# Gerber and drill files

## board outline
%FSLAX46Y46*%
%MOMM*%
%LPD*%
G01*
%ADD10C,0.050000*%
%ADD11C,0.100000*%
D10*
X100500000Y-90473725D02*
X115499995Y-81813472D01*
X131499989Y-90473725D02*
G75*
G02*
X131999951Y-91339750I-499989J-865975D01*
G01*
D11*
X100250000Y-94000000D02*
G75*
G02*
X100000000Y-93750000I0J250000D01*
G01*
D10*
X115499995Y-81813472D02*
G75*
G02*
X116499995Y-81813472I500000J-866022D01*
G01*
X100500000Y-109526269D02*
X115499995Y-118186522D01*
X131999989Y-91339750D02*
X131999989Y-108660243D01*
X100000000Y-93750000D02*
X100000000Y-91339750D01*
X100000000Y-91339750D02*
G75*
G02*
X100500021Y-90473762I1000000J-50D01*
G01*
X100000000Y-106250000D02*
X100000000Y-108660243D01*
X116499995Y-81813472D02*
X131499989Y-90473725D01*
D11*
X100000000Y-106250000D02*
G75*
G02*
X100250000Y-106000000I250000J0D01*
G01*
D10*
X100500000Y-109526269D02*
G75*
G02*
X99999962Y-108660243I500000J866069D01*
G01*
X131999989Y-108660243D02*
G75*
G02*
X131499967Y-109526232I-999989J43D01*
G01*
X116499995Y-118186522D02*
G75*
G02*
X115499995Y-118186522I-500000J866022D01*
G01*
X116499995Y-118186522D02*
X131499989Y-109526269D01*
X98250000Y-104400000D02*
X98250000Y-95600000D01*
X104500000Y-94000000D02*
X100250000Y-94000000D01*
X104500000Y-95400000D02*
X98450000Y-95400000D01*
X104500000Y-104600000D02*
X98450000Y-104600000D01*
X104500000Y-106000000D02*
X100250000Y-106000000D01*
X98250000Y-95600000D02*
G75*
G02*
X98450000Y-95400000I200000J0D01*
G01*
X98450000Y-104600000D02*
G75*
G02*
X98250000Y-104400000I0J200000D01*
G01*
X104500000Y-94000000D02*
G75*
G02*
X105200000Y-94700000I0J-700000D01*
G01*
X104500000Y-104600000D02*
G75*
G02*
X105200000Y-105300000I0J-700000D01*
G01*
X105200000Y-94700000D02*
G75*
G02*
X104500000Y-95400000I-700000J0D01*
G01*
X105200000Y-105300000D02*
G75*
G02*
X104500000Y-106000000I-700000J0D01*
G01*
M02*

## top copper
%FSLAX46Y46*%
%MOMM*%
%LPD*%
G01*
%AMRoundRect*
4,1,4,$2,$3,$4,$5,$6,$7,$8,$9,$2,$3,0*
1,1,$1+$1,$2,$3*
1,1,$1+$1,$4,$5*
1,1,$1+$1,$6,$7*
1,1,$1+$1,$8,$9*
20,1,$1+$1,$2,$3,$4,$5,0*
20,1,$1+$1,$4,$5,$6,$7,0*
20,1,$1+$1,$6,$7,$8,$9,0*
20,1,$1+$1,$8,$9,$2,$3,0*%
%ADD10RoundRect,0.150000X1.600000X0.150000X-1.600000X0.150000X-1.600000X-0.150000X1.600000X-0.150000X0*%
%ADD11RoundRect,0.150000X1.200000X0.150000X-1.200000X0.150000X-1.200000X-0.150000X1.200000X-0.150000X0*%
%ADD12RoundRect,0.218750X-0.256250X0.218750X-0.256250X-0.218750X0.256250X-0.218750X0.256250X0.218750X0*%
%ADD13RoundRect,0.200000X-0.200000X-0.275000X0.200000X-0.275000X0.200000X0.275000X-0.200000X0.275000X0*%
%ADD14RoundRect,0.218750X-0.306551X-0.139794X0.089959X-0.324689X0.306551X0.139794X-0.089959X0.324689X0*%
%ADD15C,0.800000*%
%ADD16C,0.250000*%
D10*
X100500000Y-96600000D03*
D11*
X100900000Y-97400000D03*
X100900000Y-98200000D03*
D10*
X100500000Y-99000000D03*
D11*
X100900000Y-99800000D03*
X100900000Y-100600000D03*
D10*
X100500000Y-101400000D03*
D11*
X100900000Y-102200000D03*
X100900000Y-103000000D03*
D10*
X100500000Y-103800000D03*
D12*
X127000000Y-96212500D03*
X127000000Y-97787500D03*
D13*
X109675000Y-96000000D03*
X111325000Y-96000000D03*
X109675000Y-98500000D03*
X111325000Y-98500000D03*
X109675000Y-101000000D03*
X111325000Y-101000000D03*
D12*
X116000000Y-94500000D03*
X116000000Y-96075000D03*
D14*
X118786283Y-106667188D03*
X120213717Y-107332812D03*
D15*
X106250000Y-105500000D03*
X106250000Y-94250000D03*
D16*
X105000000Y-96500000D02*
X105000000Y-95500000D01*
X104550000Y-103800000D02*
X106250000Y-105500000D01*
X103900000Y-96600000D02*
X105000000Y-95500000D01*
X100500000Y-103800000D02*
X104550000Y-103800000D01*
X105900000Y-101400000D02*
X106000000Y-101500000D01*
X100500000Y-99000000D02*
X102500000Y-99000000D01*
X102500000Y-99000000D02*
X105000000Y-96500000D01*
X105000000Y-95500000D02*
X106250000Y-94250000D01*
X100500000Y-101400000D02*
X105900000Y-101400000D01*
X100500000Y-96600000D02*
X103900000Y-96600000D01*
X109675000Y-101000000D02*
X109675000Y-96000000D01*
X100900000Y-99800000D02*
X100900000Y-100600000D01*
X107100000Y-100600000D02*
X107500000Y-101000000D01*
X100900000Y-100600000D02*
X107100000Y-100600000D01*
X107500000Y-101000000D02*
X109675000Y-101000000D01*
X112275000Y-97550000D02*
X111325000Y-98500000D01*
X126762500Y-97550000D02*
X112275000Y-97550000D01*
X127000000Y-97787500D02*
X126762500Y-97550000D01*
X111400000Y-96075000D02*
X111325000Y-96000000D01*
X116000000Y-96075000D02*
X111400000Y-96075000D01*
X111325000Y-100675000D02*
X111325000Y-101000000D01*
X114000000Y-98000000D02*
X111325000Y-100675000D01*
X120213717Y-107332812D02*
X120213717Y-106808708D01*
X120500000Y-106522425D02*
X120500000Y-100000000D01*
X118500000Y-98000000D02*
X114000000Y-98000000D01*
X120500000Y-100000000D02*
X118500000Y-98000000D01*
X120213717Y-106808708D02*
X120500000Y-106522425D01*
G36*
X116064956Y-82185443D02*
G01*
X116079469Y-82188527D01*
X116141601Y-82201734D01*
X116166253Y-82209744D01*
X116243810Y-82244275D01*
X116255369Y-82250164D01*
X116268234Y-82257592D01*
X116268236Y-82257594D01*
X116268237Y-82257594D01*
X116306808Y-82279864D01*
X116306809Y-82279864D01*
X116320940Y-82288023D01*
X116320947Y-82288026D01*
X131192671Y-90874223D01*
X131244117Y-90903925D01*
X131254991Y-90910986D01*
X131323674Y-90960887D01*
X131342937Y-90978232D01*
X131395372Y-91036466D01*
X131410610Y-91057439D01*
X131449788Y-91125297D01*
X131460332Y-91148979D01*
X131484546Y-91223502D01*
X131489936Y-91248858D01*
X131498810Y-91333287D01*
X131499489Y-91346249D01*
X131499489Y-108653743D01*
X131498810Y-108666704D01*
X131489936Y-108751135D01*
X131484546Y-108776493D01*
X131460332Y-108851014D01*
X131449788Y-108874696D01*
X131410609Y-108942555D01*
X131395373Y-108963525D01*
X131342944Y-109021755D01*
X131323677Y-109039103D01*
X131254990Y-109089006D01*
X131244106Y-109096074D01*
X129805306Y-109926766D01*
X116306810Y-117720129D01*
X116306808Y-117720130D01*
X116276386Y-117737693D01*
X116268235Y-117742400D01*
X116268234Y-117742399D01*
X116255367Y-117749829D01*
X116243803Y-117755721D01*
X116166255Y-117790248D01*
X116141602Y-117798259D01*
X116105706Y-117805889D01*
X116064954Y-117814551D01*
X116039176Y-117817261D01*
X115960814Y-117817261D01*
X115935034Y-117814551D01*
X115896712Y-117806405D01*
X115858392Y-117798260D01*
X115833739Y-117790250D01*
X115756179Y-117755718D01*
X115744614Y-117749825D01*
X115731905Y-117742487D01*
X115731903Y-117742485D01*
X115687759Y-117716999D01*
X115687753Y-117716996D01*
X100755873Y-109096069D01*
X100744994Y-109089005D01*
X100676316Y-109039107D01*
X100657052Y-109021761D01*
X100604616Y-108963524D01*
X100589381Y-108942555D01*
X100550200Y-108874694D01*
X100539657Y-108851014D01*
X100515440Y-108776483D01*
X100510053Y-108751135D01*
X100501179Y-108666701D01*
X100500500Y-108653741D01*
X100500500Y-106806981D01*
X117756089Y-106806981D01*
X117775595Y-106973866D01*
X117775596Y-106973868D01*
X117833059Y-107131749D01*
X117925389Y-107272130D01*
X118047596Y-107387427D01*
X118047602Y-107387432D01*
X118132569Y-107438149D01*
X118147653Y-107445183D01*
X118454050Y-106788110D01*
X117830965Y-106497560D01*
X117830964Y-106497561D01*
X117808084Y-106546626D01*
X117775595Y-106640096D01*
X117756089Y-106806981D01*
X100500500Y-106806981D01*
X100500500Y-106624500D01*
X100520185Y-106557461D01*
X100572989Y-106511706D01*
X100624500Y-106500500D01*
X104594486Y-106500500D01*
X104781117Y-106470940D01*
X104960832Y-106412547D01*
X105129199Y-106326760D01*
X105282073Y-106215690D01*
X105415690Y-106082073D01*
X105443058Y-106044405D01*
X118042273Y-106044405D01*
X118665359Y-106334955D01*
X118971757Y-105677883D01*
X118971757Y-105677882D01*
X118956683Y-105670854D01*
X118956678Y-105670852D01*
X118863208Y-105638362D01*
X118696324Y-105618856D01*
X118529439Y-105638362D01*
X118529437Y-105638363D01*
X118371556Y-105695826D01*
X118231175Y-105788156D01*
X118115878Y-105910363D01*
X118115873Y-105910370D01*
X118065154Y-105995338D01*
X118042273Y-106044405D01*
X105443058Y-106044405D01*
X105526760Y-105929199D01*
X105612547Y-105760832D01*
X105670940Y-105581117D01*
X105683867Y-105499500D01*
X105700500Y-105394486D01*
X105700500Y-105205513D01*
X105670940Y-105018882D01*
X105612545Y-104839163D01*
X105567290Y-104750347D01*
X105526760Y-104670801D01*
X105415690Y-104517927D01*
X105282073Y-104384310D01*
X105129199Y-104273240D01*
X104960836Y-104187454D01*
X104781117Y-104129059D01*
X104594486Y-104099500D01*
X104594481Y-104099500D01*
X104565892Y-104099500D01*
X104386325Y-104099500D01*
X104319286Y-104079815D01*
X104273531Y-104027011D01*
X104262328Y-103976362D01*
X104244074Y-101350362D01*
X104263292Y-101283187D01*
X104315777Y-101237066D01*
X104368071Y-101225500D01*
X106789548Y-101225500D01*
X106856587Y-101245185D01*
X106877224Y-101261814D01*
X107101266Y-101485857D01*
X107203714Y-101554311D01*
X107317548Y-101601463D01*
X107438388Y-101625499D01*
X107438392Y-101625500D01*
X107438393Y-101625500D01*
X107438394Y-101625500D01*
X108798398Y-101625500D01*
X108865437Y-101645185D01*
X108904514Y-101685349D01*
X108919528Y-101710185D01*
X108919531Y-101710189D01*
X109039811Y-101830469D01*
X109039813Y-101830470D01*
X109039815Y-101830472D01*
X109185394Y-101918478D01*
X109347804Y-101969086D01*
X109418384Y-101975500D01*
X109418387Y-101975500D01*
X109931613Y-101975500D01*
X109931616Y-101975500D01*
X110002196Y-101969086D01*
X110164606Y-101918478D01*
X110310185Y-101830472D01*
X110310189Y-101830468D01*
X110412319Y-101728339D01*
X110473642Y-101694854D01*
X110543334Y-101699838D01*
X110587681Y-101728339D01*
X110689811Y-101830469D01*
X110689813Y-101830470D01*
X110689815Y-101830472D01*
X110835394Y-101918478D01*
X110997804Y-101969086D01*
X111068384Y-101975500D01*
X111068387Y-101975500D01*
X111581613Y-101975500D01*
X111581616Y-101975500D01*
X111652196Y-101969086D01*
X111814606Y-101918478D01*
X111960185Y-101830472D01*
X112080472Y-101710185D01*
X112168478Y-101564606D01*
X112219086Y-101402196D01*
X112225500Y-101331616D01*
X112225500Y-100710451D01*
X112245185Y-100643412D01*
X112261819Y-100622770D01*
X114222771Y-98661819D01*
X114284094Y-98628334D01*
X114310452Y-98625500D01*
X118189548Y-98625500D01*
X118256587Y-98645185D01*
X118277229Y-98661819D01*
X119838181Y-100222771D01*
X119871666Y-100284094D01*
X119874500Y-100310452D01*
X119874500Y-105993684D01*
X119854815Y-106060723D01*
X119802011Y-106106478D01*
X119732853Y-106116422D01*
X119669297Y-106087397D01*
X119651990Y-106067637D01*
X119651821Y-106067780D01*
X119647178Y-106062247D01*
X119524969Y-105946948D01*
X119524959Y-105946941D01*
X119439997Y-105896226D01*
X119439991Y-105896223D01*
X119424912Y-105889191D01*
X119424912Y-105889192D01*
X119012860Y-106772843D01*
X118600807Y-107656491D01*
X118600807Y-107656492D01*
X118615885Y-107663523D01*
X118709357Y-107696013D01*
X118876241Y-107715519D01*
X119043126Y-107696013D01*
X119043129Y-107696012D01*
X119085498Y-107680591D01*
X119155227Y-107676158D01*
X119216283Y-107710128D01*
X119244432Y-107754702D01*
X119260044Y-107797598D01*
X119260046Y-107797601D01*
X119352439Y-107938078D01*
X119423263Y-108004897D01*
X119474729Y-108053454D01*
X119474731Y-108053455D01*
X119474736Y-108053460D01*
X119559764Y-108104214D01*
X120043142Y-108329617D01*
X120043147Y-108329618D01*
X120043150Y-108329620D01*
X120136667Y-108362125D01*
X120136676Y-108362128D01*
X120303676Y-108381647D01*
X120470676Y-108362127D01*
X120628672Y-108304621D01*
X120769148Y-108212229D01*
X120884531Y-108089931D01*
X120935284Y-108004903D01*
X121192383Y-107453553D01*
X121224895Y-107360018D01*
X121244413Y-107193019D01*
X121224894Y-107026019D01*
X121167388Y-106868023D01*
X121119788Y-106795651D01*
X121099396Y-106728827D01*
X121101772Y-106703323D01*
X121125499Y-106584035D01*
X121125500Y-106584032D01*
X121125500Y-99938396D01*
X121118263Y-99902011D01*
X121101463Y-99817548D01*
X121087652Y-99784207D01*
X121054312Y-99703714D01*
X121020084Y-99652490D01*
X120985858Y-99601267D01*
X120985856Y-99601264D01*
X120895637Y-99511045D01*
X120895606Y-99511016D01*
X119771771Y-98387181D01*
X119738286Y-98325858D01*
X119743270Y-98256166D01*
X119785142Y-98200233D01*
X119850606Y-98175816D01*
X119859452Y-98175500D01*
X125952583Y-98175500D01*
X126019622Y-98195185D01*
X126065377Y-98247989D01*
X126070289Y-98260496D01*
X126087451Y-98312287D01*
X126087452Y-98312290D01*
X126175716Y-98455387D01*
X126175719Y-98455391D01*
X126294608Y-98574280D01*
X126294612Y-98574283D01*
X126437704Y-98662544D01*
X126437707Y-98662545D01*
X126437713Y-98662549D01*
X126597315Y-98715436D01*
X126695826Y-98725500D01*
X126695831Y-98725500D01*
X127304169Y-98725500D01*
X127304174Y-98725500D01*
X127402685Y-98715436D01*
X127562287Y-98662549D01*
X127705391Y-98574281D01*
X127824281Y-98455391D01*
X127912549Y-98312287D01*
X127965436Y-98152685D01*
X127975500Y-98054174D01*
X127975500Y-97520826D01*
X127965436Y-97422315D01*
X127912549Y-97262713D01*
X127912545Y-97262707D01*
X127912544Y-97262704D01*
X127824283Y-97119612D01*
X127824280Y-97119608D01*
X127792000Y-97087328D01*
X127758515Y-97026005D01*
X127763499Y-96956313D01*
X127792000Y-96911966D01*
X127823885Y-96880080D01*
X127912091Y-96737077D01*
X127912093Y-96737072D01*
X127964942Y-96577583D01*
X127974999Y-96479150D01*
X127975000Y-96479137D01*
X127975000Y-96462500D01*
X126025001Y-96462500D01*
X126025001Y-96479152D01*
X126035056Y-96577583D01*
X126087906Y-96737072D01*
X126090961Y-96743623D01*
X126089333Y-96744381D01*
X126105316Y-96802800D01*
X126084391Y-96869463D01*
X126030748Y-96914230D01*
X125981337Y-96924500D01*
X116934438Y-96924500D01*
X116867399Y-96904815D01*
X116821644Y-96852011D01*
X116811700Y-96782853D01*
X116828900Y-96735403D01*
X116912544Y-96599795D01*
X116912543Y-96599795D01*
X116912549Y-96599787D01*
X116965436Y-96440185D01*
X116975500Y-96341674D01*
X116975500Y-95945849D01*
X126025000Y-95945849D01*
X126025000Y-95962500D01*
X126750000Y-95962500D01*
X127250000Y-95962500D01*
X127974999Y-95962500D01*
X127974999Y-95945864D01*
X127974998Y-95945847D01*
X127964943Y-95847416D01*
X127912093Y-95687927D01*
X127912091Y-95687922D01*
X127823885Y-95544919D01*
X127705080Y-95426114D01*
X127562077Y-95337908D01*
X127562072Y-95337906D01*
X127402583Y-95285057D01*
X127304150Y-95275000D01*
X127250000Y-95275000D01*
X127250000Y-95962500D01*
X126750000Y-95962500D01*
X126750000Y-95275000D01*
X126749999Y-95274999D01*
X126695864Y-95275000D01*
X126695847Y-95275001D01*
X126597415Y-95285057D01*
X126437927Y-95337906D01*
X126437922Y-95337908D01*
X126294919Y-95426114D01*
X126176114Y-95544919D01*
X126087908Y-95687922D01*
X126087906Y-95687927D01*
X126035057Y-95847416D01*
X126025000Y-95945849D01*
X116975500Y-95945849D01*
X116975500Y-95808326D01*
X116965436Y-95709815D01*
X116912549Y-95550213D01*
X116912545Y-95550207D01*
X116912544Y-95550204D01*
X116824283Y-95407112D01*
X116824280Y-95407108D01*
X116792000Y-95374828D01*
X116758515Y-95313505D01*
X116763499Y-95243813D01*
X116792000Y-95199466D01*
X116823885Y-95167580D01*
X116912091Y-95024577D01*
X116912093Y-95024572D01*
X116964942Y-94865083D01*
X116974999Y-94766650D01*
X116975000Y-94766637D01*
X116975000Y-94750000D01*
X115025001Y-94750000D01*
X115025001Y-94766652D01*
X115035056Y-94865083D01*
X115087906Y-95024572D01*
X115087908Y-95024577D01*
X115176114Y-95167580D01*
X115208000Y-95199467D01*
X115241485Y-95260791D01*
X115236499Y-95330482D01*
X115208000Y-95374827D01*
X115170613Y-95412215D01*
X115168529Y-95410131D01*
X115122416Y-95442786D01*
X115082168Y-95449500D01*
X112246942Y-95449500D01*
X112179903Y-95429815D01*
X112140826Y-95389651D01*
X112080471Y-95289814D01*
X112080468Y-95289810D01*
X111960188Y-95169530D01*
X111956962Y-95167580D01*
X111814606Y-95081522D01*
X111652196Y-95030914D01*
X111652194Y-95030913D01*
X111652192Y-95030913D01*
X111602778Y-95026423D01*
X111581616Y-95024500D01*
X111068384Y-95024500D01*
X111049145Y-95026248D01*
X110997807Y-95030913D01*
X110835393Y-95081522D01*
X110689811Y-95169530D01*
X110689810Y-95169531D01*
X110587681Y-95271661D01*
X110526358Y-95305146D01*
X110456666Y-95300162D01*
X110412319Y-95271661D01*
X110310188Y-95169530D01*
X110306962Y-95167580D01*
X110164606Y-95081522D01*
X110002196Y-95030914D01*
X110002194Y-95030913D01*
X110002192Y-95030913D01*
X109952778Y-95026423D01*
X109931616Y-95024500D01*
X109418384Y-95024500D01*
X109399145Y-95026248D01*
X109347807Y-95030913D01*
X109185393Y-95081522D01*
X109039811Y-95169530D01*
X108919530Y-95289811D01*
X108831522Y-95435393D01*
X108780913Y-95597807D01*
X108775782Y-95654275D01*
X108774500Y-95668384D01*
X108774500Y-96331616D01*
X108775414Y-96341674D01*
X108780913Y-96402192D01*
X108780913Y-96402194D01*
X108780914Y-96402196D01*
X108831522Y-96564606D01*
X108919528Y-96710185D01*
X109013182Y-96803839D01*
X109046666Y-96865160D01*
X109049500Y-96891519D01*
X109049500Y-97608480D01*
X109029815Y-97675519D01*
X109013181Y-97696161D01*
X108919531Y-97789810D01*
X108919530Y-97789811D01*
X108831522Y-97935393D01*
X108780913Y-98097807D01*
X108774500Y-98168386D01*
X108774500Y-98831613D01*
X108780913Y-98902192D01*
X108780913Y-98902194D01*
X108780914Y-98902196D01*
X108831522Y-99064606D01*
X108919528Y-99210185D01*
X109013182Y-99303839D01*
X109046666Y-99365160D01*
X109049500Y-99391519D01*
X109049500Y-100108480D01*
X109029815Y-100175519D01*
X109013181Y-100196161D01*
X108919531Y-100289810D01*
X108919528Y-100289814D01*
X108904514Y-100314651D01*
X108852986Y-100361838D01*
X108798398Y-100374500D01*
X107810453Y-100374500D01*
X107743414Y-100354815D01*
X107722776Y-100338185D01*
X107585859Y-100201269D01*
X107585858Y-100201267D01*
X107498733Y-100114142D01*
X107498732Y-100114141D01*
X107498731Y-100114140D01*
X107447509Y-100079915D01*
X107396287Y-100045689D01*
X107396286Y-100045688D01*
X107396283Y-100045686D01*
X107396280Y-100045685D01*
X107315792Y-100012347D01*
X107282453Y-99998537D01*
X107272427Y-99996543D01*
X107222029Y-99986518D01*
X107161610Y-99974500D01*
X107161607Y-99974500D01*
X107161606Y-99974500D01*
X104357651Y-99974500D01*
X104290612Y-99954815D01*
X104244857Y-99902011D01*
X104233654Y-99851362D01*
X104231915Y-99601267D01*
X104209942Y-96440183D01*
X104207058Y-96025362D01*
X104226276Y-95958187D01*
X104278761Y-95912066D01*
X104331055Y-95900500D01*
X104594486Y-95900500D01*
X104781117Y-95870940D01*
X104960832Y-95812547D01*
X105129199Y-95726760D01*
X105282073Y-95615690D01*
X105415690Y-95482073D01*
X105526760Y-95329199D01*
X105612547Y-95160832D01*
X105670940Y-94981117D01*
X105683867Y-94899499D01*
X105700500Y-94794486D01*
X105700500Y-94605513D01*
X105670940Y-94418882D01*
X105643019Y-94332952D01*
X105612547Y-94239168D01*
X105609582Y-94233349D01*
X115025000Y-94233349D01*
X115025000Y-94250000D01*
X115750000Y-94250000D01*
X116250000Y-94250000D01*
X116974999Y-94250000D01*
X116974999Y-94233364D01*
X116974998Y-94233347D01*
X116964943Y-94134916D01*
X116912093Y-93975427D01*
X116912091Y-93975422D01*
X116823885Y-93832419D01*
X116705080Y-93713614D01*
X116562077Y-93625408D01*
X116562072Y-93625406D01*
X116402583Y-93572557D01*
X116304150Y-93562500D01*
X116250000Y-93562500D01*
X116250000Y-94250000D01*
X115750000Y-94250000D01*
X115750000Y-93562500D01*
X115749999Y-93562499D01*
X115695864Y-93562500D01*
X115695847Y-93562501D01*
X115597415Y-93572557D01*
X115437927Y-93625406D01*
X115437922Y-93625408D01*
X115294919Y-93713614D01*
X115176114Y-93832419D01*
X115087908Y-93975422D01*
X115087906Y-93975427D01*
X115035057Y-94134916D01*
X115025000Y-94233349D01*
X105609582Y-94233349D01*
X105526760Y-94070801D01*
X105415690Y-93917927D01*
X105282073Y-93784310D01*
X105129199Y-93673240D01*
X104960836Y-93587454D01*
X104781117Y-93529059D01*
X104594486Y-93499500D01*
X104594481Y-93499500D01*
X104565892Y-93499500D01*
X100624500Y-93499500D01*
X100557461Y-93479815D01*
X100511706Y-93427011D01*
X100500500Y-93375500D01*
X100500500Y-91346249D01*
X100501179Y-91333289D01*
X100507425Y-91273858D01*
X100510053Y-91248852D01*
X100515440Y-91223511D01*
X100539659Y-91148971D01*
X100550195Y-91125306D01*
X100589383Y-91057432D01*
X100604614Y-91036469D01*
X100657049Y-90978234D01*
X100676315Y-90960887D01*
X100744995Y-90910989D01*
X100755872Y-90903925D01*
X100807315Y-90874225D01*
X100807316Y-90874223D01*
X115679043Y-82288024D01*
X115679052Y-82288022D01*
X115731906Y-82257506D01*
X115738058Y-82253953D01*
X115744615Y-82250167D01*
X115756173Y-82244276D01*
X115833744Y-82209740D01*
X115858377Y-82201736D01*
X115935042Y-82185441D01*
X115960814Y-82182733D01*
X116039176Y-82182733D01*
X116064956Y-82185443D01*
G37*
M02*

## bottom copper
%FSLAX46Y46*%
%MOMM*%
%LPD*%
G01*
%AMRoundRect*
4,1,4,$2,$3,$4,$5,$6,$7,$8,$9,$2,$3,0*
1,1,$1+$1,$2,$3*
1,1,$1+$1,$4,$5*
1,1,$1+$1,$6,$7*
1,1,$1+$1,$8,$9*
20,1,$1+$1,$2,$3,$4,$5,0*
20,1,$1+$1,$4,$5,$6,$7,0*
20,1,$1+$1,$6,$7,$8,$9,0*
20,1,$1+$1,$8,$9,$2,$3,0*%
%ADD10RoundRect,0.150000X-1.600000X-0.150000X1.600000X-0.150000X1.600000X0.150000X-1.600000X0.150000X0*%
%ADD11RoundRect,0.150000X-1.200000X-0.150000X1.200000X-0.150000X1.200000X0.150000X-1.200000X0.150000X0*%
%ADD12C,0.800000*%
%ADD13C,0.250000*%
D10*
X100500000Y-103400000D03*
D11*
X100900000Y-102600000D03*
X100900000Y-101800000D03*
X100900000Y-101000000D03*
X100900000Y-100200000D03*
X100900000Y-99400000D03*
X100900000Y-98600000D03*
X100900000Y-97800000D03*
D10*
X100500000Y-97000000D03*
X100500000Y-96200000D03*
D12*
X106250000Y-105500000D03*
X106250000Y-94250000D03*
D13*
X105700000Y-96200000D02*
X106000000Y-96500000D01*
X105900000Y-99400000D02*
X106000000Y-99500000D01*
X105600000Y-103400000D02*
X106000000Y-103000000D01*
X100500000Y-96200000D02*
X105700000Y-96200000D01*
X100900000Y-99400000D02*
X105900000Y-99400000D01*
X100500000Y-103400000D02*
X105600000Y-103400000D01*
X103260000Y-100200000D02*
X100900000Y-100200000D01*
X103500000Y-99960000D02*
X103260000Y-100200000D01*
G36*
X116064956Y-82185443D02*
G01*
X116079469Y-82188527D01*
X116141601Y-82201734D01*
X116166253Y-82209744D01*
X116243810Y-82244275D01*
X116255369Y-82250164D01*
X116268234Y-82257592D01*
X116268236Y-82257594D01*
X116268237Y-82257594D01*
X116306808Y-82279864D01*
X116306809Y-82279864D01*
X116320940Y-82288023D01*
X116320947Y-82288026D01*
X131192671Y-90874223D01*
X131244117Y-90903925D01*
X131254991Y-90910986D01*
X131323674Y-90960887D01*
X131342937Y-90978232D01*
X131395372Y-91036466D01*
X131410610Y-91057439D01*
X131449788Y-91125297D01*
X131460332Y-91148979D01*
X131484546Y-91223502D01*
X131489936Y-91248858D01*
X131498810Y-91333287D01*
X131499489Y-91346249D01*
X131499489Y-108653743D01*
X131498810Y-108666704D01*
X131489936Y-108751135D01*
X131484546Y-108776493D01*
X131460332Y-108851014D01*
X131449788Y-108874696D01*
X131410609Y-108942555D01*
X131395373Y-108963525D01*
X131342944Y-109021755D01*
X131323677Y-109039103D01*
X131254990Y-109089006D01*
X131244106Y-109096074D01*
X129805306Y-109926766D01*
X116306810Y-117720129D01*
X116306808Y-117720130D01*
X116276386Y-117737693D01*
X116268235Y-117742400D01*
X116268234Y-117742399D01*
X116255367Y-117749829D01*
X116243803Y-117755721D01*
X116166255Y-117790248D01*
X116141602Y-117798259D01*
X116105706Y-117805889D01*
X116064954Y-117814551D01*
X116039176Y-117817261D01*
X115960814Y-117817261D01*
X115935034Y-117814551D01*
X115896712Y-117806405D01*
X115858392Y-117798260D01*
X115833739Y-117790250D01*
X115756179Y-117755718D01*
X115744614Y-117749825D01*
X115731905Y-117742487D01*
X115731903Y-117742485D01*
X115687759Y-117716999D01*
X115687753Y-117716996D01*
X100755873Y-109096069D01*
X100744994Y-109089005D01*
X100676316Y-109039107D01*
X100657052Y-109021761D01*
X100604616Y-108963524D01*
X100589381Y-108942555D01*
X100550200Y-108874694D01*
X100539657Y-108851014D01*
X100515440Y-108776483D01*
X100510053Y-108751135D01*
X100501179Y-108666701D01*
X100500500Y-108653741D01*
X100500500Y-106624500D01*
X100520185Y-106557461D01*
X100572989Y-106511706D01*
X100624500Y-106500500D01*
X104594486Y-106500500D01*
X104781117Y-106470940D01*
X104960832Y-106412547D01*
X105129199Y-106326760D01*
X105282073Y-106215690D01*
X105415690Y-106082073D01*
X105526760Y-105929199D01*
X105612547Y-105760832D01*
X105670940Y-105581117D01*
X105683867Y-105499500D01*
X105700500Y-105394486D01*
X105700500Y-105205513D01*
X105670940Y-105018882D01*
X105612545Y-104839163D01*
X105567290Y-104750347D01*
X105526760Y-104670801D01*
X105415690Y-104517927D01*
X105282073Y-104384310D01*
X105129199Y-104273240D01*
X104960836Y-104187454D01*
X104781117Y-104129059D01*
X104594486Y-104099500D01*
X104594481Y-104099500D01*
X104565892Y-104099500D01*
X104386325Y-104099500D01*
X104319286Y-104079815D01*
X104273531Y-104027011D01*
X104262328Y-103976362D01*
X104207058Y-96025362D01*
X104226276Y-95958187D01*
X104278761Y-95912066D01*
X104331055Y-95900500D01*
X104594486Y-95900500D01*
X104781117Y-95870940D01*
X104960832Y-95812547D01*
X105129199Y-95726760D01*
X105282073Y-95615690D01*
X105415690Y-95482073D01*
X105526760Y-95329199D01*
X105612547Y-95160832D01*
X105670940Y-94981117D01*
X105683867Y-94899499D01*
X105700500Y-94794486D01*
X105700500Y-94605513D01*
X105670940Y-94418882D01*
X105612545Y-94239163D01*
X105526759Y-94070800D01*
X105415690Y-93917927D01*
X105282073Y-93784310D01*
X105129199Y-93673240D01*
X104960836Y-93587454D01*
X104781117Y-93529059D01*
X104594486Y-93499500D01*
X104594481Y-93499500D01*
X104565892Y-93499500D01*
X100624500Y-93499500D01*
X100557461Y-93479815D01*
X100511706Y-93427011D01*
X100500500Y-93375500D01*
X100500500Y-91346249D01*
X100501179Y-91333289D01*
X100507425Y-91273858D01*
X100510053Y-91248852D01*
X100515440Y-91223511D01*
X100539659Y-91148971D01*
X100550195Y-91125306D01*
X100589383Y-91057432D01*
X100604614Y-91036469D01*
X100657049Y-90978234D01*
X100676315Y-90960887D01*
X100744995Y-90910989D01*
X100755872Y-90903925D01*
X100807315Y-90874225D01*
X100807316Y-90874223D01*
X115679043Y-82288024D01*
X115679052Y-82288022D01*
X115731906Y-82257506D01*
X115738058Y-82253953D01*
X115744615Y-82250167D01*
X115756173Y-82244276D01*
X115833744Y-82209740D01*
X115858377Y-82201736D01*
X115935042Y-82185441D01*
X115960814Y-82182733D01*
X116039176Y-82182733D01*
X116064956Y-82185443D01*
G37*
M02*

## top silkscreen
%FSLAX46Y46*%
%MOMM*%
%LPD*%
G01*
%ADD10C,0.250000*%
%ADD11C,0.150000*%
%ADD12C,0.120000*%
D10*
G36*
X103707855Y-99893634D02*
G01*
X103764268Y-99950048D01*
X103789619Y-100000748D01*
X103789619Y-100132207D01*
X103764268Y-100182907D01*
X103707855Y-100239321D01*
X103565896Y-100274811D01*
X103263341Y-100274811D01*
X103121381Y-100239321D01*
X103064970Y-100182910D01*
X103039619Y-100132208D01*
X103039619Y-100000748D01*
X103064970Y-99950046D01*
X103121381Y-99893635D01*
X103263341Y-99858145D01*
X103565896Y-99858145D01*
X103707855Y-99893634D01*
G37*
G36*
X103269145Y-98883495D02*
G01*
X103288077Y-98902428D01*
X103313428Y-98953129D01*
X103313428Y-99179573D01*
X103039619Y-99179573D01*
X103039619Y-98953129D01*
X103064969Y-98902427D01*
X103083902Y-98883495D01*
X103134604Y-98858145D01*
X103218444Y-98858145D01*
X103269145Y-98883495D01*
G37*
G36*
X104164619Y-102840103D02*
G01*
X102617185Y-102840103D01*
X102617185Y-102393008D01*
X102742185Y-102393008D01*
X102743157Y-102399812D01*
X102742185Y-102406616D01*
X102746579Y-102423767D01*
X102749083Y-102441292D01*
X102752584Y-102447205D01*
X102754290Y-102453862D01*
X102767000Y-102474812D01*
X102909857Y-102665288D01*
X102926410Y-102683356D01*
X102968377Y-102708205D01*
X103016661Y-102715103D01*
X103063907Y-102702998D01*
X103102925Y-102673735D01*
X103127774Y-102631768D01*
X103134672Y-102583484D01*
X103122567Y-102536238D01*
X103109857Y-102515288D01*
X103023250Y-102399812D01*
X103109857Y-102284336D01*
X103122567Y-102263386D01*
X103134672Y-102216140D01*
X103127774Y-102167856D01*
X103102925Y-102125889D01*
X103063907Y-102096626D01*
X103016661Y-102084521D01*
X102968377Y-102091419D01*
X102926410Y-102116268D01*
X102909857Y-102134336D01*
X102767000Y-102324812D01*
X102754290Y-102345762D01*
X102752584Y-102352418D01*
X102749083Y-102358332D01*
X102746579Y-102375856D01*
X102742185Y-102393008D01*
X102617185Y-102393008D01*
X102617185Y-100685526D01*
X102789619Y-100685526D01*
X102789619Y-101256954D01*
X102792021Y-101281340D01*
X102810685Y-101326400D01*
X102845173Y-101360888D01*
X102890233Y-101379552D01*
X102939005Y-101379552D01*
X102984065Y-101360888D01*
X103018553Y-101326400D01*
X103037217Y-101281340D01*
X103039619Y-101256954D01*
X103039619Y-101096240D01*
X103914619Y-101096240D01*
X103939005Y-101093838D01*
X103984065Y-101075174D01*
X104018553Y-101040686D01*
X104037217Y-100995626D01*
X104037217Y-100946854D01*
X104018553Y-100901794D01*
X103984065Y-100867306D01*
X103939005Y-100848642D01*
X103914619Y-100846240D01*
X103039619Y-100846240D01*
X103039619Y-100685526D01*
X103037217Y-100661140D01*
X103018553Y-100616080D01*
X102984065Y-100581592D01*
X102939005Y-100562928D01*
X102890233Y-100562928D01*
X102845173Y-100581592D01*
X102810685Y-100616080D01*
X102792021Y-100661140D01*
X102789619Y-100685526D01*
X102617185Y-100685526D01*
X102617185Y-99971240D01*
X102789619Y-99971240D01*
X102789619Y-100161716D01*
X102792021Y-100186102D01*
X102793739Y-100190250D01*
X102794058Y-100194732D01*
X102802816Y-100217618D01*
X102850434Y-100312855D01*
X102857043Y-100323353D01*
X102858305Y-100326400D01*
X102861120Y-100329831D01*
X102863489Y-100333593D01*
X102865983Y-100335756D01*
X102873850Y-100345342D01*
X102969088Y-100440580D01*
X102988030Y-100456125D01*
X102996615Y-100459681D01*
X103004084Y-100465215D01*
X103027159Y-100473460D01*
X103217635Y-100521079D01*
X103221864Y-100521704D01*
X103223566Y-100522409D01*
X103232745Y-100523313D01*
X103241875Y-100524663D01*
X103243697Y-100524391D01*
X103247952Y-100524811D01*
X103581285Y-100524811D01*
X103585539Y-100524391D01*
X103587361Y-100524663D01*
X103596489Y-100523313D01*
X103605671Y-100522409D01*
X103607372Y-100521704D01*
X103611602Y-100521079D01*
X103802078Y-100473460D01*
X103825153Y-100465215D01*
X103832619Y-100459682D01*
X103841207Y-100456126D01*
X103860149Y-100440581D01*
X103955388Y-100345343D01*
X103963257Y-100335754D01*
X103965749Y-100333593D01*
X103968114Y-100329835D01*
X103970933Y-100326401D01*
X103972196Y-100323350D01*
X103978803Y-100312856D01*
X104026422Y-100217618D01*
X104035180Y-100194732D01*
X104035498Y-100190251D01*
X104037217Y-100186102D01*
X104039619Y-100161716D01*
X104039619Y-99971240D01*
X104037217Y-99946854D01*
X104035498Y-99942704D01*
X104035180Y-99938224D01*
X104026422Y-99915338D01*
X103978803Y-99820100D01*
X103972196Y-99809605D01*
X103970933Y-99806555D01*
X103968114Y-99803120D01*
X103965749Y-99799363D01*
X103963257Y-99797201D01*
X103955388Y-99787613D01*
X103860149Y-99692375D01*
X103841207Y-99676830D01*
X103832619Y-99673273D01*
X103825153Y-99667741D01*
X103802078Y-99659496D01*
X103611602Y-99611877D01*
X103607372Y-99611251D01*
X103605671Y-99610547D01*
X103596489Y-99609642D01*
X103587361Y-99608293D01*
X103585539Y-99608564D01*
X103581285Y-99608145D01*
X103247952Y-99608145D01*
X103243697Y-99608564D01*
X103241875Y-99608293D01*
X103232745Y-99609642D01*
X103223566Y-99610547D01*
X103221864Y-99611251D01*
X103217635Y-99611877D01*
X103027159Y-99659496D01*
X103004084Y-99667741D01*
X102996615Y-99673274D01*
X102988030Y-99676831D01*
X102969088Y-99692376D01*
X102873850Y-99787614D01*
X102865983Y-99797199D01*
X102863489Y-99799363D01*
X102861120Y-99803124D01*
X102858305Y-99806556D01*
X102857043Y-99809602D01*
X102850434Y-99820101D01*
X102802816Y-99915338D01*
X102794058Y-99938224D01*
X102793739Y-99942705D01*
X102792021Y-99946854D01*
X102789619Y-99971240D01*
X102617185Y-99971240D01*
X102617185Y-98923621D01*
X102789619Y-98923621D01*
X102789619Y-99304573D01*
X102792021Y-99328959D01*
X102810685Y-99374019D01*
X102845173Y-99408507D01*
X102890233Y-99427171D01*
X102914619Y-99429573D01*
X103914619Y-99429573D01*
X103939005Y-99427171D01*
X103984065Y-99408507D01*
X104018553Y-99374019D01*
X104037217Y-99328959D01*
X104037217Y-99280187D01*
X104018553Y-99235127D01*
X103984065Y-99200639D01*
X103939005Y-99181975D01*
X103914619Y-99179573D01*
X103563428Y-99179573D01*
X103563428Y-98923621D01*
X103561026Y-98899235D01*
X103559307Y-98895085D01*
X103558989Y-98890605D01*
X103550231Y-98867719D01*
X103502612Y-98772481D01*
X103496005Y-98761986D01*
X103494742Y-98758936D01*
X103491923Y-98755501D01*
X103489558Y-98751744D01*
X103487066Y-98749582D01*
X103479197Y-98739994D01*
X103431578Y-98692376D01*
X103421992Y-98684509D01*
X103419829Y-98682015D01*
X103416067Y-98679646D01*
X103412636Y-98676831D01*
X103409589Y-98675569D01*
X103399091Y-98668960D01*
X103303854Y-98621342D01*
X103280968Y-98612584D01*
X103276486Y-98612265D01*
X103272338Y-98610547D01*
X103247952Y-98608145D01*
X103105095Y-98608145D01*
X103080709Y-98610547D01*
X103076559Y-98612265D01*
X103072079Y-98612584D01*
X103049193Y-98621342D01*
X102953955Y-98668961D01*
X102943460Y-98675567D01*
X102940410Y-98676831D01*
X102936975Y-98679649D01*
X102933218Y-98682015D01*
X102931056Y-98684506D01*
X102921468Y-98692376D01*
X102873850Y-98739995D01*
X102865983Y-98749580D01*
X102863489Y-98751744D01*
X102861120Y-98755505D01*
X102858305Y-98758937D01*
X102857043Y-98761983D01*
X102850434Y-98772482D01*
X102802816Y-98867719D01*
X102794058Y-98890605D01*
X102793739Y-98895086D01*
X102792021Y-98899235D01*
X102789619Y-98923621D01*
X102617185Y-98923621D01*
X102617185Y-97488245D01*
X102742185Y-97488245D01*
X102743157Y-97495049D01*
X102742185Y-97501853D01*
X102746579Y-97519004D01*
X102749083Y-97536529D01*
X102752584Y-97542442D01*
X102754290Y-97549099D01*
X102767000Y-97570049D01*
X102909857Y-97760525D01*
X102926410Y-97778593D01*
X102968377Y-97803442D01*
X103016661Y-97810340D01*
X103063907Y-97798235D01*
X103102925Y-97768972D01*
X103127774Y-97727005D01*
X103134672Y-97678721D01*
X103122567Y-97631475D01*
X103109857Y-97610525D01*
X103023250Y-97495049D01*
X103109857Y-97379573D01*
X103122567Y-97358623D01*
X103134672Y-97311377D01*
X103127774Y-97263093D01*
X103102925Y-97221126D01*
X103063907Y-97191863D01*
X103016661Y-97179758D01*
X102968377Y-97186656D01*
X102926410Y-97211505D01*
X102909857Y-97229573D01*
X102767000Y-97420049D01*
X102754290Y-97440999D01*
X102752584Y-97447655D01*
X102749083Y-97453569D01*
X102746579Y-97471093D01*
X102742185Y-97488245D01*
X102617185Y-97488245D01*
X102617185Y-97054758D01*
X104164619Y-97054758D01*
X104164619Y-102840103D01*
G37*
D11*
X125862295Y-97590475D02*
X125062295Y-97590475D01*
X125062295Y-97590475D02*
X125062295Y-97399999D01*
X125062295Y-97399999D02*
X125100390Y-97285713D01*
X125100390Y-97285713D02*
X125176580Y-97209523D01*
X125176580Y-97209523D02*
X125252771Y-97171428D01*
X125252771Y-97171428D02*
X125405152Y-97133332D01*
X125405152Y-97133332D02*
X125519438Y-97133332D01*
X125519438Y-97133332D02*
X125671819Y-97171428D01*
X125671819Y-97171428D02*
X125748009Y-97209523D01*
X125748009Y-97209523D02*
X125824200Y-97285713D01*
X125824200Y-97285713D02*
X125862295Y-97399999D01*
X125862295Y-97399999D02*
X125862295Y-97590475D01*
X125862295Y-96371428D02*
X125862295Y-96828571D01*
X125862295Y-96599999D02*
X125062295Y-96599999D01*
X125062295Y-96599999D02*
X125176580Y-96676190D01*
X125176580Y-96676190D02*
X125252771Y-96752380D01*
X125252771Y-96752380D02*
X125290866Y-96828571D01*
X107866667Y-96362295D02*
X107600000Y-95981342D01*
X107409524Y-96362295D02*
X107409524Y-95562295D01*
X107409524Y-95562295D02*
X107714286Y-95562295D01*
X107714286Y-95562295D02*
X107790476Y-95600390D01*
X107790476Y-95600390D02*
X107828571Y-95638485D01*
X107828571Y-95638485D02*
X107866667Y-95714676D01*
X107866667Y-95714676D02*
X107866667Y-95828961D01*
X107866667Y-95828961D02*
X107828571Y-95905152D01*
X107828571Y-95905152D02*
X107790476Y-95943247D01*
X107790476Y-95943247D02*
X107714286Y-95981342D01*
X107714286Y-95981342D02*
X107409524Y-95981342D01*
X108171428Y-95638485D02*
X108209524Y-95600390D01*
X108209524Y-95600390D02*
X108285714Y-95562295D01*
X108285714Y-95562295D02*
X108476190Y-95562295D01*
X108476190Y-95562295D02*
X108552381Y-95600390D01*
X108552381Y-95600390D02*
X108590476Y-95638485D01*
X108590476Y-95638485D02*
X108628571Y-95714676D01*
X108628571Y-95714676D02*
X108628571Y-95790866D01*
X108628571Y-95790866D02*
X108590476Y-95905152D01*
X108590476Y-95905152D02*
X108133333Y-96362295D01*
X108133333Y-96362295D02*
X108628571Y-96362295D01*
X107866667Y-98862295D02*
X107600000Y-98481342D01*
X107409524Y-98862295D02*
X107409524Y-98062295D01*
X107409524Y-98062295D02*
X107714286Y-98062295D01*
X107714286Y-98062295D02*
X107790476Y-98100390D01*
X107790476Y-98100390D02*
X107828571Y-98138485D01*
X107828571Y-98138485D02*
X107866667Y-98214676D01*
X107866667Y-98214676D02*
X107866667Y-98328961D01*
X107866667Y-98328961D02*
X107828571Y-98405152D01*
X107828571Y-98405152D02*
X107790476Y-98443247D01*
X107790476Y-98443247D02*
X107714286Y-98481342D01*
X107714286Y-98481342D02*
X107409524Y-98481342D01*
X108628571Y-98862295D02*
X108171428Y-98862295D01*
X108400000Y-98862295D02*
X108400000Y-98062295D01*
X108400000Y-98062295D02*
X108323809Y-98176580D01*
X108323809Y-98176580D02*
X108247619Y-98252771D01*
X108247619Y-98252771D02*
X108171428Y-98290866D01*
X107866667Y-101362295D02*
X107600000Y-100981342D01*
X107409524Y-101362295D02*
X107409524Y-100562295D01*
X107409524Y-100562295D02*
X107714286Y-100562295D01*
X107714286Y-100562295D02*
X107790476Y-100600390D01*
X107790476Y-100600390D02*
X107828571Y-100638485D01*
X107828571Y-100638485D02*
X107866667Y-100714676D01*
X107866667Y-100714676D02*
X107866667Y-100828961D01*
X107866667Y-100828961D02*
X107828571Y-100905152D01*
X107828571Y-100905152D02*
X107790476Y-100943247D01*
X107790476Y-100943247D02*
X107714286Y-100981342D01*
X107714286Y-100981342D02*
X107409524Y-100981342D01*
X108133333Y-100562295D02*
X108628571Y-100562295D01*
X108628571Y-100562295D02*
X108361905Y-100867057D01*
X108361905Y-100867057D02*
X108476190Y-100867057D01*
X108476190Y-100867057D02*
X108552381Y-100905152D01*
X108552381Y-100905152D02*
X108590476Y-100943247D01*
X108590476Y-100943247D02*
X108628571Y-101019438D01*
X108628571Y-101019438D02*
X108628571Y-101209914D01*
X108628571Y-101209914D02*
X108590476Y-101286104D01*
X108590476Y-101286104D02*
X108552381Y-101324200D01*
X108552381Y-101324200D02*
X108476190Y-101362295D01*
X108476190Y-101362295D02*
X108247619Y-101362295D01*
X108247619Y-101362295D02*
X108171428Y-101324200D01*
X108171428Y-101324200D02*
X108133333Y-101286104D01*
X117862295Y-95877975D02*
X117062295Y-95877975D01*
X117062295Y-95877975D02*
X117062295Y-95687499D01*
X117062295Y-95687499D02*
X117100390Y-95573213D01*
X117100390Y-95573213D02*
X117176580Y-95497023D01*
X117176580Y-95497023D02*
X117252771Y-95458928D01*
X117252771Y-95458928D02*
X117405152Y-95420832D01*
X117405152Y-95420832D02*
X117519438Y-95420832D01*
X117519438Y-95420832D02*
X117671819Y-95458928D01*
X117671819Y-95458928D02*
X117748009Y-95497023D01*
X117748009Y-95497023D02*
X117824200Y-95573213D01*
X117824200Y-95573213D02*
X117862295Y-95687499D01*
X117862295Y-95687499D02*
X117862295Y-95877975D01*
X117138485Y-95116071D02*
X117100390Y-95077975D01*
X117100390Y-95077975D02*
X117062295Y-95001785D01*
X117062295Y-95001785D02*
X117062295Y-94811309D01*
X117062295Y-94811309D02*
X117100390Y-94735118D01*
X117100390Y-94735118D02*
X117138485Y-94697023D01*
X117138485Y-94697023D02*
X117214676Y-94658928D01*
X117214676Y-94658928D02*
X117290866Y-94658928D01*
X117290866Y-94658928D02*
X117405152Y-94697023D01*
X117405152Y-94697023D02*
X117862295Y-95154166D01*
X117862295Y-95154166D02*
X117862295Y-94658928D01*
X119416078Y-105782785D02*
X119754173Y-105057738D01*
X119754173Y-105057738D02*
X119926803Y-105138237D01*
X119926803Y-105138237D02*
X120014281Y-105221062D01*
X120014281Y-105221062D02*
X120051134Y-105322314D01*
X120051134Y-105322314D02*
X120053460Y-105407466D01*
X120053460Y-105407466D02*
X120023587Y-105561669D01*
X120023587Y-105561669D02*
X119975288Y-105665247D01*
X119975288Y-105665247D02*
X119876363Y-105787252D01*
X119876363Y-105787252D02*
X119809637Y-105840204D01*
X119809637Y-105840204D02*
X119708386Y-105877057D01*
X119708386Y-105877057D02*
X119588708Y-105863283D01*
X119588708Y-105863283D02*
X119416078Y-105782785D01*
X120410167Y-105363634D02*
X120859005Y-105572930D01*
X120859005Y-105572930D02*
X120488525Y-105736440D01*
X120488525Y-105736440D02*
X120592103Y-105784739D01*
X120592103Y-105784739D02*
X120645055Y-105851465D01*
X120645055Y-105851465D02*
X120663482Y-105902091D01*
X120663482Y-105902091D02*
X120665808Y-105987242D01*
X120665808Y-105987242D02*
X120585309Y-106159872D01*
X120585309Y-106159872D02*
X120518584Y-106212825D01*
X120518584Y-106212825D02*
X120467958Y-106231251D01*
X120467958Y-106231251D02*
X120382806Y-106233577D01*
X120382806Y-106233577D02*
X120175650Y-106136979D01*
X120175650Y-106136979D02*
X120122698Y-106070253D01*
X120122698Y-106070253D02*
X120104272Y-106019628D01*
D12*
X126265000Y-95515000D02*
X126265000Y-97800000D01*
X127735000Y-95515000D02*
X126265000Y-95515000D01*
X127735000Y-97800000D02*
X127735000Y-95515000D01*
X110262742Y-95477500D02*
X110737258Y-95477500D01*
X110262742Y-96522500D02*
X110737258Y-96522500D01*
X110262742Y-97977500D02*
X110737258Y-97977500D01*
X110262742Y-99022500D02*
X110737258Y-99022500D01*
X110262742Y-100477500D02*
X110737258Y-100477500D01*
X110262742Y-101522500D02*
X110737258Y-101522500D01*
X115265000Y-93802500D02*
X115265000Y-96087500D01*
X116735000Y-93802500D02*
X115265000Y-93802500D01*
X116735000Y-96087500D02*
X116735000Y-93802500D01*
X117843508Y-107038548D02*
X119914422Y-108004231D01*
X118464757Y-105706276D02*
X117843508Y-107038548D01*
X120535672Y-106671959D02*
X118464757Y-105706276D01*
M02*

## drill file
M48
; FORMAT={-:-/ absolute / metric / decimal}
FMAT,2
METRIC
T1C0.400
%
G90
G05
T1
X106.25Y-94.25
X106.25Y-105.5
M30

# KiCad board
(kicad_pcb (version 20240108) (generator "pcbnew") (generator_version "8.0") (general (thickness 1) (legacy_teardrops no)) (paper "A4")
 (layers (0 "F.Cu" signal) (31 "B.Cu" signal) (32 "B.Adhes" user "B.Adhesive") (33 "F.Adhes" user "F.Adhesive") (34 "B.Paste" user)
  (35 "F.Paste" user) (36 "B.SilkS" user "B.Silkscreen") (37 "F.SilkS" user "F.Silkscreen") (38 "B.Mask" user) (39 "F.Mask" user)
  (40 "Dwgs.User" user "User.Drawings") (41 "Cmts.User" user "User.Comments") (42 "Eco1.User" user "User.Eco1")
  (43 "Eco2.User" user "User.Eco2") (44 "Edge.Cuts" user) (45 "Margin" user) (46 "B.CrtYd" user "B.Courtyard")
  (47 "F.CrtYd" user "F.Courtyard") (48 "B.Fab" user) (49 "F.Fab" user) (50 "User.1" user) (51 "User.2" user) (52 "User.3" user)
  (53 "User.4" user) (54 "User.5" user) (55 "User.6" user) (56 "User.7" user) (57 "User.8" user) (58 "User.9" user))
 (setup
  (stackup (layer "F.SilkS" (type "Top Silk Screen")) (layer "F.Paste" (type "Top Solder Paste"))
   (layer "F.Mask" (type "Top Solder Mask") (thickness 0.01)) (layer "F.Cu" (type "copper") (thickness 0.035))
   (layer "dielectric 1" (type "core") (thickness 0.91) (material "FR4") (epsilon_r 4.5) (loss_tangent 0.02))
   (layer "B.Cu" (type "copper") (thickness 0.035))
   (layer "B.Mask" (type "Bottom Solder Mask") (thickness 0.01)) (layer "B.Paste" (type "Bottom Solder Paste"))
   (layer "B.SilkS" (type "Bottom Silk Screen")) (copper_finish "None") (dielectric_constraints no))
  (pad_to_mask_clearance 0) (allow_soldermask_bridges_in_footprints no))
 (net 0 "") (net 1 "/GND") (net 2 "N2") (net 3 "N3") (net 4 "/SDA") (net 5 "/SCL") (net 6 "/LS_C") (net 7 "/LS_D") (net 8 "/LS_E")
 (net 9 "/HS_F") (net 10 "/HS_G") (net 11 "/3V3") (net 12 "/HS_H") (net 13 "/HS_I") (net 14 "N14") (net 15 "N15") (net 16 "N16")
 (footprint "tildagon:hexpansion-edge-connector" (layer "F.Cu") (at 98.25 100)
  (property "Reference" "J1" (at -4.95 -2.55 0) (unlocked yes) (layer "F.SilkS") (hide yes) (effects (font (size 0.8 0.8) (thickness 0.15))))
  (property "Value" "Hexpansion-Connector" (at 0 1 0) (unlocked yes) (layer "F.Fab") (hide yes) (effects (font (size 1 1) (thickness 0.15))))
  (fp_line (start 0 4.4) (end 0 -4.4) (stroke (width 0.05) (type solid)) (layer "Edge.Cuts"))
  (fp_line (start 6.25 -6) (end 2 -6) (stroke (width 0.05) (type solid)) (layer "Edge.Cuts"))
  (fp_line (start 6.25 -4.6) (end 0.2 -4.6) (stroke (width 0.05) (type solid)) (layer "Edge.Cuts"))
  (fp_line (start 6.25 4.6) (end 0.2 4.6) (stroke (width 0.05) (type solid)) (layer "Edge.Cuts"))
  (fp_line (start 6.25 6) (end 2 6) (stroke (width 0.05) (type solid)) (layer "Edge.Cuts"))
  (fp_arc (start 0 -4.4) (mid 0.058579 -4.541421) (end 0.2 -4.6) (stroke (width 0.05) (type default)) (layer "Edge.Cuts"))
  (fp_arc (start 0.2 4.6) (mid 0.058579 4.541421) (end 0 4.4) (stroke (width 0.05) (type default)) (layer "Edge.Cuts"))
  (fp_arc (start 6.25 -6) (mid 6.744975 -5.794975) (end 6.95 -5.3) (stroke (width 0.05) (type default)) (layer "Edge.Cuts"))
  (fp_arc (start 6.25 4.6) (mid 6.744975 4.805025) (end 6.95 5.3) (stroke (width 0.05) (type default)) (layer "Edge.Cuts"))
  (fp_arc (start 6.95 -5.3) (mid 6.744975 -4.805025) (end 6.25 -4.6) (stroke (width 0.05) (type default)) (layer "Edge.Cuts"))
  (fp_arc (start 6.95 5.3) (mid 6.744975 5.794975) (end 6.25 6) (stroke (width 0.05) (type default)) (layer "Edge.Cuts"))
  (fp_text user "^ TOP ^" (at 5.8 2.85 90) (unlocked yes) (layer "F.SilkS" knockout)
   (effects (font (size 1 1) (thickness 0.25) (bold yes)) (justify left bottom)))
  (pad "1" smd roundrect (at 2.25 3.4) (size 3.5 0.6) (layers "B.Cu" "B.Mask") (roundrect_rratio 0.25) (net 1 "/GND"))
  (pad "2" smd roundrect (at 2.65 2.6) (size 2.7 0.6) (layers "B.Cu" "B.Mask") (roundrect_rratio 0.25) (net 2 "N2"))
  (pad "3" smd roundrect (at 2.65 1.8) (size 2.7 0.6) (layers "B.Cu" "B.Mask") (roundrect_rratio 0.25) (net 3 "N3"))
  (pad "4" smd roundrect (at 2.65 1) (size 2.7 0.6) (layers "B.Cu" "B.Mask") (roundrect_rratio 0.25) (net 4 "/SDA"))
  (pad "5" smd roundrect (at 2.65 0.2) (size 2.7 0.6) (layers "B.Cu" "B.Mask") (roundrect_rratio 0.25) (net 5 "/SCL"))
  (pad "6" smd roundrect (at 2.65 -0.6) (size 2.7 0.6) (layers "B.Cu" "B.Mask") (roundrect_rratio 0.25) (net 1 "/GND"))
  (pad "7" smd roundrect (at 2.65 -1.4) (size 2.7 0.6) (layers "B.Cu" "B.Mask") (roundrect_rratio 0.25) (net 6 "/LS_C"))
  (pad "8" smd roundrect (at 2.65 -2.2) (size 2.7 0.6) (layers "B.Cu" "B.Mask") (roundrect_rratio 0.25) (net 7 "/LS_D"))
  (pad "9" smd roundrect (at 2.25 -3) (size 3.5 0.6) (layers "B.Cu" "B.Mask") (roundrect_rratio 0.25) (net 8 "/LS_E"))
  (pad "10" smd roundrect (at 2.25 -3.8) (size 3.5 0.6) (layers "B.Cu" "B.Mask") (roundrect_rratio 0.25) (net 1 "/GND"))
  (pad "11" smd roundrect (at 2.25 -3.4 180) (size 3.5 0.6) (layers "F.Cu" "F.Mask") (roundrect_rratio 0.25) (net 1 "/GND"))
  (pad "12" smd roundrect (at 2.65 -2.6 180) (size 2.7 0.6) (layers "F.Cu" "F.Mask") (roundrect_rratio 0.25) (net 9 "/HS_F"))
  (pad "13" smd roundrect (at 2.65 -1.8 180) (size 2.7 0.6) (layers "F.Cu" "F.Mask") (roundrect_rratio 0.25) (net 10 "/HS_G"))
  (pad "14" smd roundrect (at 2.25 -1 180) (size 3.5 0.6) (layers "F.Cu" "F.Mask") (roundrect_rratio 0.25) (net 1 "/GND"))
  (pad "15" smd roundrect (at 2.65 -0.2 180) (size 2.7 0.6) (layers "F.Cu" "F.Mask") (roundrect_rratio 0.25) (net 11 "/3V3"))
  (pad "16" smd roundrect (at 2.65 0.6 180) (size 2.7 0.6) (layers "F.Cu" "F.Mask") (roundrect_rratio 0.25) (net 11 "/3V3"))
  (pad "17" smd roundrect (at 2.25 1.4 180) (size 3.5 0.6) (layers "F.Cu" "F.Mask") (roundrect_rratio 0.25) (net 1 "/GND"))
  (pad "18" smd roundrect (at 2.65 2.2 180) (size 2.7 0.6) (layers "F.Cu" "F.Mask") (roundrect_rratio 0.25) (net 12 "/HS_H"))
  (pad "19" smd roundrect (at 2.65 3 180) (size 2.7 0.6) (layers "F.Cu" "F.Mask") (roundrect_rratio 0.25) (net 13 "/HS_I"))
  (pad "20" smd roundrect (at 2.25 3.8 180) (size 3.5 0.6) (layers "F.Cu" "F.Mask") (roundrect_rratio 0.25) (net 1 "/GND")))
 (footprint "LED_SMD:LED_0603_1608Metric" (layer "F.Cu") (at 127 97 -90)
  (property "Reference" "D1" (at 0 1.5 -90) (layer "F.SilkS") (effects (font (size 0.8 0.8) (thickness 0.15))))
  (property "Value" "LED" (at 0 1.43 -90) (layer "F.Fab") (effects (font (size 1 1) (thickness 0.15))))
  (fp_line (start -1.485 0.735) (end 0.8 0.735) (stroke (width 0.12) (type solid)) (layer "F.SilkS"))
  (fp_line (start -1.485 -0.735) (end -1.485 0.735) (stroke (width 0.12) (type solid)) (layer "F.SilkS"))
  (fp_line (start 0.8 -0.735) (end -1.485 -0.735) (stroke (width 0.12) (type solid)) (layer "F.SilkS"))
  (pad "1" smd roundrect (at -0.7875 0 270) (size 0.875 0.95) (layers "F.Cu" "F.Paste" "F.Mask") (roundrect_rratio 0.25) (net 1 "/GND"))
  (pad "2" smd roundrect (at 0.7875 0 270) (size 0.875 0.95) (layers "F.Cu" "F.Paste" "F.Mask") (roundrect_rratio 0.25) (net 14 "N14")))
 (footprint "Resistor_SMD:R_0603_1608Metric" (layer "F.Cu") (at 110.5 96)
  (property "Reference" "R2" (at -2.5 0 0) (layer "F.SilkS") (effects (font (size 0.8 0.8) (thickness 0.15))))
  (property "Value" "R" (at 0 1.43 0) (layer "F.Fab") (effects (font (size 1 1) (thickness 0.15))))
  (fp_line (start -0.237258 -0.5225) (end 0.237258 -0.5225) (stroke (width 0.12) (type solid)) (layer "F.SilkS"))
  (fp_line (start -0.237258 0.5225) (end 0.237258 0.5225) (stroke (width 0.12) (type solid)) (layer "F.SilkS"))
  (pad "1" smd roundrect (at -0.825 0) (size 0.8 0.95) (layers "F.Cu" "F.Paste" "F.Mask") (roundrect_rratio 0.25) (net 11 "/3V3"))
  (pad "2" smd roundrect (at 0.825 0) (size 0.8 0.95) (layers "F.Cu" "F.Paste" "F.Mask") (roundrect_rratio 0.25) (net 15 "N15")))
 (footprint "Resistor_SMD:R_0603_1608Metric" (layer "F.Cu") (at 110.5 98.5)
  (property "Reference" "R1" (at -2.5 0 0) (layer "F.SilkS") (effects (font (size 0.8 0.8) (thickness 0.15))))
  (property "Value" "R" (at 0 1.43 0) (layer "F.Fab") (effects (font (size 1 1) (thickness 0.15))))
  (fp_line (start -0.237258 -0.5225) (end 0.237258 -0.5225) (stroke (width 0.12) (type solid)) (layer "F.SilkS"))
  (fp_line (start -0.237258 0.5225) (end 0.237258 0.5225) (stroke (width 0.12) (type solid)) (layer "F.SilkS"))
  (pad "1" smd roundrect (at -0.825 0) (size 0.8 0.95) (layers "F.Cu" "F.Paste" "F.Mask") (roundrect_rratio 0.25) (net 11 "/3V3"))
  (pad "2" smd roundrect (at 0.825 0) (size 0.8 0.95) (layers "F.Cu" "F.Paste" "F.Mask") (roundrect_rratio 0.25) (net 14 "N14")))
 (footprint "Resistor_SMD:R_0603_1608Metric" (layer "F.Cu") (at 110.5 101)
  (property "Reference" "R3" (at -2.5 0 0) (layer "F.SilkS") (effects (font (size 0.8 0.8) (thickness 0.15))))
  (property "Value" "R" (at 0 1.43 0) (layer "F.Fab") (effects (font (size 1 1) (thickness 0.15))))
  (fp_line (start -0.237258 -0.5225) (end 0.237258 -0.5225) (stroke (width 0.12) (type solid)) (layer "F.SilkS"))
  (fp_line (start -0.237258 0.5225) (end 0.237258 0.5225) (stroke (width 0.12) (type solid)) (layer "F.SilkS"))
  (pad "1" smd roundrect (at -0.825 0) (size 0.8 0.95) (layers "F.Cu" "F.Paste" "F.Mask") (roundrect_rratio 0.25) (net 11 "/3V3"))
  (pad "2" smd roundrect (at 0.825 0) (size 0.8 0.95) (layers "F.Cu" "F.Paste" "F.Mask") (roundrect_rratio 0.25) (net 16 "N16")))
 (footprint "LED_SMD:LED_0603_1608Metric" (layer "F.Cu") (at 116 95.2875 -90)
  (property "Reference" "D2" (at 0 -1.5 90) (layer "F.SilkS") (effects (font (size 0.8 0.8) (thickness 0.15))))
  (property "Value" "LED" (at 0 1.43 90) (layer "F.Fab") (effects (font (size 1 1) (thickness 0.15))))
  (fp_line (start -1.485 0.735) (end 0.8 0.735) (stroke (width 0.12) (type solid)) (layer "F.SilkS"))
  (fp_line (start -1.485 -0.735) (end -1.485 0.735) (stroke (width 0.12) (type solid)) (layer "F.SilkS"))
  (fp_line (start 0.8 -0.735) (end -1.485 -0.735) (stroke (width 0.12) (type solid)) (layer "F.SilkS"))
  (pad "1" smd roundrect (at -0.7875 0 270) (size 0.875 0.95) (layers "F.Cu" "F.Paste" "F.Mask") (roundrect_rratio 0.25) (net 1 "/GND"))
  (pad "2" smd roundrect (at 0.7875 0 270) (size 0.875 0.95) (layers "F.Cu" "F.Paste" "F.Mask") (roundrect_rratio 0.25) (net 15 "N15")))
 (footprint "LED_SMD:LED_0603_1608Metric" (layer "F.Cu") (at 119.5 107 -25)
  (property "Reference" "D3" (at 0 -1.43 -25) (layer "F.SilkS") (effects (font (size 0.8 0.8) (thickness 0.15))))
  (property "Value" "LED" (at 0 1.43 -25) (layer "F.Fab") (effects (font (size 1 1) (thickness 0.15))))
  (fp_line (start -1.485001 0.735) (end 0.8 0.735) (stroke (width 0.12) (type solid)) (layer "F.SilkS"))
  (fp_line (start -1.485 -0.735) (end -1.485001 0.735) (stroke (width 0.12) (type solid)) (layer "F.SilkS"))
  (fp_line (start 0.800001 -0.735) (end -1.485 -0.735) (stroke (width 0.12) (type solid)) (layer "F.SilkS"))
  (pad "1" smd roundrect (at -0.7875 0 335) (size 0.875 0.95) (layers "F.Cu" "F.Paste" "F.Mask") (roundrect_rratio 0.25) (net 1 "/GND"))
  (pad "2" smd roundrect (at 0.7875 0 335) (size 0.875 0.95) (layers "F.Cu" "F.Paste" "F.Mask") (roundrect_rratio 0.25) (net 16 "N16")))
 (gr_line (start 100.5 90.473725) (end 115.499995 81.813472) (stroke (width 0.05) (type solid)) (layer "Edge.Cuts"))
 (gr_arc (start 131.499989 90.473725) (mid 131.866015 90.83975) (end 131.999989 91.33975) (stroke (width 0.05) (type solid))
  (layer "Edge.Cuts"))
 (gr_arc (start 100.25 94) (mid 100.073223 93.926777) (end 100 93.75) (stroke (width 0.1) (type default)) (layer "Edge.Cuts"))
 (gr_arc (start 115.499995 81.813472) (mid 115.999995 81.679497) (end 116.499995 81.813472) (stroke (width 0.05) (type solid))
  (layer "Edge.Cuts"))
 (gr_line (start 100.5 109.526269) (end 115.499995 118.186522) (stroke (width 0.05) (type solid)) (layer "Edge.Cuts"))
 (gr_line (start 131.999989 91.33975) (end 131.999989 108.660243) (stroke (width 0.05) (type solid)) (layer "Edge.Cuts"))
 (gr_line (start 100 93.75) (end 100 91.33975) (stroke (width 0.05) (type solid)) (layer "Edge.Cuts"))
 (gr_arc (start 100 91.33975) (mid 100.133975 90.83975) (end 100.5 90.473725) (stroke (width 0.05) (type solid)) (layer "Edge.Cuts"))
 (gr_line (start 100 106.25) (end 100 108.660243) (stroke (width 0.05) (type solid)) (layer "Edge.Cuts"))
 (gr_line (start 116.499995 81.813472) (end 131.499989 90.473725) (stroke (width 0.05) (type solid)) (layer "Edge.Cuts"))
 (gr_arc (start 100 106.25) (mid 100.073223 106.073223) (end 100.25 106) (stroke (width 0.1) (type default)) (layer "Edge.Cuts"))
 (gr_arc (start 100.5 109.526269) (mid 100.133975 109.160243) (end 100 108.660243) (stroke (width 0.05) (type solid)) (layer "Edge.Cuts"))
 (gr_arc (start 131.999989 108.660243) (mid 131.866015 109.160243) (end 131.499989 109.526269) (stroke (width 0.05) (type solid))
  (layer "Edge.Cuts"))
 (gr_arc (start 116.499995 118.186522) (mid 115.999995 118.320497) (end 115.499995 118.186522) (stroke (width 0.05) (type solid))
  (layer "Edge.Cuts"))
 (gr_line (start 116.499995 118.186522) (end 131.499989 109.526269) (stroke (width 0.05) (type solid)) (layer "Edge.Cuts"))
 (segment (start 105 96.5) (end 105 95.5) (width 0.25) (layer "F.Cu") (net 1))
 (segment (start 104.55 103.8) (end 106.25 105.5) (width 0.25) (layer "F.Cu") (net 1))
 (segment (start 103.9 96.6) (end 105 95.5) (width 0.25) (layer "F.Cu") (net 1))
 (segment (start 100.5 103.8) (end 104.55 103.8) (width 0.25) (layer "F.Cu") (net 1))
 (segment (start 105.9 101.4) (end 106 101.5) (width 0.25) (layer "F.Cu") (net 1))
 (segment (start 100.5 99) (end 102.5 99) (width 0.25) (layer "F.Cu") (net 1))
 (segment (start 102.5 99) (end 105 96.5) (width 0.25) (layer "F.Cu") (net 1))
 (segment (start 105 95.5) (end 106.25 94.25) (width 0.25) (layer "F.Cu") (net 1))
 (segment (start 100.5 101.4) (end 105.9 101.4) (width 0.25) (layer "F.Cu") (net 1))
 (segment (start 100.5 96.6) (end 103.9 96.6) (width 0.25) (layer "F.Cu") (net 1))
 (via (at 106.25 105.5) (size 0.8) (drill 0.4) (layers "F.Cu" "B.Cu") (free yes) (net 1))
 (via (at 106.25 94.25) (size 0.8) (drill 0.4) (layers "F.Cu" "B.Cu") (free yes) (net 1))
 (segment (start 105.7 96.2) (end 106 96.5) (width 0.25) (layer "B.Cu") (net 1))
 (segment (start 105.9 99.4) (end 106 99.5) (width 0.25) (layer "B.Cu") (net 1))
 (segment (start 105.6 103.4) (end 106 103) (width 0.25) (layer "B.Cu") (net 1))
 (segment (start 100.5 96.2) (end 105.7 96.2) (width 0.25) (layer "B.Cu") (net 1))
 (segment (start 100.9 99.4) (end 105.9 99.4) (width 0.25) (layer "B.Cu") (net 1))
 (segment (start 100.5 103.4) (end 105.6 103.4) (width 0.25) (layer "B.Cu") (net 1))
 (segment (start 103.26 100.2) (end 100.9 100.2) (width 0.25) (layer "B.Cu") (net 5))
 (segment (start 103.5 99.96) (end 103.26 100.2) (width 0.25) (layer "B.Cu") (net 5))
 (segment (start 109.675 101) (end 109.675 96) (width 0.25) (layer "F.Cu") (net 11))
 (segment (start 100.9 99.8) (end 100.9 100.6) (width 0.25) (layer "F.Cu") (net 11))
 (segment (start 107.1 100.6) (end 107.5 101) (width 0.25) (layer "F.Cu") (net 11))
 (segment (start 100.9 100.6) (end 107.1 100.6) (width 0.25) (layer "F.Cu") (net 11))
 (segment (start 107.5 101) (end 109.675 101) (width 0.25) (layer "F.Cu") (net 11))
 (segment (start 112.275 97.55) (end 111.325 98.5) (width 0.25) (layer "F.Cu") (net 14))
 (segment (start 126.7625 97.55) (end 112.275 97.55) (width 0.25) (layer "F.Cu") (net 14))
 (segment (start 127 97.7875) (end 126.7625 97.55) (width 0.25) (layer "F.Cu") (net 14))
 (segment (start 111.4 96.075) (end 111.325 96) (width 0.25) (layer "F.Cu") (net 15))
 (segment (start 116 96.075) (end 111.4 96.075) (width 0.25) (layer "F.Cu") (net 15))
 (segment (start 111.325 100.675) (end 111.325 101) (width 0.25) (layer "F.Cu") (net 16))
 (segment (start 114 98) (end 111.325 100.675) (width 0.25) (layer "F.Cu") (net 16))
 (segment (start 120.213717 107.332812) (end 120.213717 106.808708) (width 0.25) (layer "F.Cu") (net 16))
 (segment (start 120.5 106.522425) (end 120.5 100) (width 0.25) (layer "F.Cu") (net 16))
 (segment (start 118.5 98) (end 114 98) (width 0.25) (layer "F.Cu") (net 16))
 (segment (start 120.5 100) (end 118.5 98) (width 0.25) (layer "F.Cu") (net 16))
 (segment (start 120.213717 106.808708) (end 120.5 106.522425) (width 0.25) (layer "F.Cu") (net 16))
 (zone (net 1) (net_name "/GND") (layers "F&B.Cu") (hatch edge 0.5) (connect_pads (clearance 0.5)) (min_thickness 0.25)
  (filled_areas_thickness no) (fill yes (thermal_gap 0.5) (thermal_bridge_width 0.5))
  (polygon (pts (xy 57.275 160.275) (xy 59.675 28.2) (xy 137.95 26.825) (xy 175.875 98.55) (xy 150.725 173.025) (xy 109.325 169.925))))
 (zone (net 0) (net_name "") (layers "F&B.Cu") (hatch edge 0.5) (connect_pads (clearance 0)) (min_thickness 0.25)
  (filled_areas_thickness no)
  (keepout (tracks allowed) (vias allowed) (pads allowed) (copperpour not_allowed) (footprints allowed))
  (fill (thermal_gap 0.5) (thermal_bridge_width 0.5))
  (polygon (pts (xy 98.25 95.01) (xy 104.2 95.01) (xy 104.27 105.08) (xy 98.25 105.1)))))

